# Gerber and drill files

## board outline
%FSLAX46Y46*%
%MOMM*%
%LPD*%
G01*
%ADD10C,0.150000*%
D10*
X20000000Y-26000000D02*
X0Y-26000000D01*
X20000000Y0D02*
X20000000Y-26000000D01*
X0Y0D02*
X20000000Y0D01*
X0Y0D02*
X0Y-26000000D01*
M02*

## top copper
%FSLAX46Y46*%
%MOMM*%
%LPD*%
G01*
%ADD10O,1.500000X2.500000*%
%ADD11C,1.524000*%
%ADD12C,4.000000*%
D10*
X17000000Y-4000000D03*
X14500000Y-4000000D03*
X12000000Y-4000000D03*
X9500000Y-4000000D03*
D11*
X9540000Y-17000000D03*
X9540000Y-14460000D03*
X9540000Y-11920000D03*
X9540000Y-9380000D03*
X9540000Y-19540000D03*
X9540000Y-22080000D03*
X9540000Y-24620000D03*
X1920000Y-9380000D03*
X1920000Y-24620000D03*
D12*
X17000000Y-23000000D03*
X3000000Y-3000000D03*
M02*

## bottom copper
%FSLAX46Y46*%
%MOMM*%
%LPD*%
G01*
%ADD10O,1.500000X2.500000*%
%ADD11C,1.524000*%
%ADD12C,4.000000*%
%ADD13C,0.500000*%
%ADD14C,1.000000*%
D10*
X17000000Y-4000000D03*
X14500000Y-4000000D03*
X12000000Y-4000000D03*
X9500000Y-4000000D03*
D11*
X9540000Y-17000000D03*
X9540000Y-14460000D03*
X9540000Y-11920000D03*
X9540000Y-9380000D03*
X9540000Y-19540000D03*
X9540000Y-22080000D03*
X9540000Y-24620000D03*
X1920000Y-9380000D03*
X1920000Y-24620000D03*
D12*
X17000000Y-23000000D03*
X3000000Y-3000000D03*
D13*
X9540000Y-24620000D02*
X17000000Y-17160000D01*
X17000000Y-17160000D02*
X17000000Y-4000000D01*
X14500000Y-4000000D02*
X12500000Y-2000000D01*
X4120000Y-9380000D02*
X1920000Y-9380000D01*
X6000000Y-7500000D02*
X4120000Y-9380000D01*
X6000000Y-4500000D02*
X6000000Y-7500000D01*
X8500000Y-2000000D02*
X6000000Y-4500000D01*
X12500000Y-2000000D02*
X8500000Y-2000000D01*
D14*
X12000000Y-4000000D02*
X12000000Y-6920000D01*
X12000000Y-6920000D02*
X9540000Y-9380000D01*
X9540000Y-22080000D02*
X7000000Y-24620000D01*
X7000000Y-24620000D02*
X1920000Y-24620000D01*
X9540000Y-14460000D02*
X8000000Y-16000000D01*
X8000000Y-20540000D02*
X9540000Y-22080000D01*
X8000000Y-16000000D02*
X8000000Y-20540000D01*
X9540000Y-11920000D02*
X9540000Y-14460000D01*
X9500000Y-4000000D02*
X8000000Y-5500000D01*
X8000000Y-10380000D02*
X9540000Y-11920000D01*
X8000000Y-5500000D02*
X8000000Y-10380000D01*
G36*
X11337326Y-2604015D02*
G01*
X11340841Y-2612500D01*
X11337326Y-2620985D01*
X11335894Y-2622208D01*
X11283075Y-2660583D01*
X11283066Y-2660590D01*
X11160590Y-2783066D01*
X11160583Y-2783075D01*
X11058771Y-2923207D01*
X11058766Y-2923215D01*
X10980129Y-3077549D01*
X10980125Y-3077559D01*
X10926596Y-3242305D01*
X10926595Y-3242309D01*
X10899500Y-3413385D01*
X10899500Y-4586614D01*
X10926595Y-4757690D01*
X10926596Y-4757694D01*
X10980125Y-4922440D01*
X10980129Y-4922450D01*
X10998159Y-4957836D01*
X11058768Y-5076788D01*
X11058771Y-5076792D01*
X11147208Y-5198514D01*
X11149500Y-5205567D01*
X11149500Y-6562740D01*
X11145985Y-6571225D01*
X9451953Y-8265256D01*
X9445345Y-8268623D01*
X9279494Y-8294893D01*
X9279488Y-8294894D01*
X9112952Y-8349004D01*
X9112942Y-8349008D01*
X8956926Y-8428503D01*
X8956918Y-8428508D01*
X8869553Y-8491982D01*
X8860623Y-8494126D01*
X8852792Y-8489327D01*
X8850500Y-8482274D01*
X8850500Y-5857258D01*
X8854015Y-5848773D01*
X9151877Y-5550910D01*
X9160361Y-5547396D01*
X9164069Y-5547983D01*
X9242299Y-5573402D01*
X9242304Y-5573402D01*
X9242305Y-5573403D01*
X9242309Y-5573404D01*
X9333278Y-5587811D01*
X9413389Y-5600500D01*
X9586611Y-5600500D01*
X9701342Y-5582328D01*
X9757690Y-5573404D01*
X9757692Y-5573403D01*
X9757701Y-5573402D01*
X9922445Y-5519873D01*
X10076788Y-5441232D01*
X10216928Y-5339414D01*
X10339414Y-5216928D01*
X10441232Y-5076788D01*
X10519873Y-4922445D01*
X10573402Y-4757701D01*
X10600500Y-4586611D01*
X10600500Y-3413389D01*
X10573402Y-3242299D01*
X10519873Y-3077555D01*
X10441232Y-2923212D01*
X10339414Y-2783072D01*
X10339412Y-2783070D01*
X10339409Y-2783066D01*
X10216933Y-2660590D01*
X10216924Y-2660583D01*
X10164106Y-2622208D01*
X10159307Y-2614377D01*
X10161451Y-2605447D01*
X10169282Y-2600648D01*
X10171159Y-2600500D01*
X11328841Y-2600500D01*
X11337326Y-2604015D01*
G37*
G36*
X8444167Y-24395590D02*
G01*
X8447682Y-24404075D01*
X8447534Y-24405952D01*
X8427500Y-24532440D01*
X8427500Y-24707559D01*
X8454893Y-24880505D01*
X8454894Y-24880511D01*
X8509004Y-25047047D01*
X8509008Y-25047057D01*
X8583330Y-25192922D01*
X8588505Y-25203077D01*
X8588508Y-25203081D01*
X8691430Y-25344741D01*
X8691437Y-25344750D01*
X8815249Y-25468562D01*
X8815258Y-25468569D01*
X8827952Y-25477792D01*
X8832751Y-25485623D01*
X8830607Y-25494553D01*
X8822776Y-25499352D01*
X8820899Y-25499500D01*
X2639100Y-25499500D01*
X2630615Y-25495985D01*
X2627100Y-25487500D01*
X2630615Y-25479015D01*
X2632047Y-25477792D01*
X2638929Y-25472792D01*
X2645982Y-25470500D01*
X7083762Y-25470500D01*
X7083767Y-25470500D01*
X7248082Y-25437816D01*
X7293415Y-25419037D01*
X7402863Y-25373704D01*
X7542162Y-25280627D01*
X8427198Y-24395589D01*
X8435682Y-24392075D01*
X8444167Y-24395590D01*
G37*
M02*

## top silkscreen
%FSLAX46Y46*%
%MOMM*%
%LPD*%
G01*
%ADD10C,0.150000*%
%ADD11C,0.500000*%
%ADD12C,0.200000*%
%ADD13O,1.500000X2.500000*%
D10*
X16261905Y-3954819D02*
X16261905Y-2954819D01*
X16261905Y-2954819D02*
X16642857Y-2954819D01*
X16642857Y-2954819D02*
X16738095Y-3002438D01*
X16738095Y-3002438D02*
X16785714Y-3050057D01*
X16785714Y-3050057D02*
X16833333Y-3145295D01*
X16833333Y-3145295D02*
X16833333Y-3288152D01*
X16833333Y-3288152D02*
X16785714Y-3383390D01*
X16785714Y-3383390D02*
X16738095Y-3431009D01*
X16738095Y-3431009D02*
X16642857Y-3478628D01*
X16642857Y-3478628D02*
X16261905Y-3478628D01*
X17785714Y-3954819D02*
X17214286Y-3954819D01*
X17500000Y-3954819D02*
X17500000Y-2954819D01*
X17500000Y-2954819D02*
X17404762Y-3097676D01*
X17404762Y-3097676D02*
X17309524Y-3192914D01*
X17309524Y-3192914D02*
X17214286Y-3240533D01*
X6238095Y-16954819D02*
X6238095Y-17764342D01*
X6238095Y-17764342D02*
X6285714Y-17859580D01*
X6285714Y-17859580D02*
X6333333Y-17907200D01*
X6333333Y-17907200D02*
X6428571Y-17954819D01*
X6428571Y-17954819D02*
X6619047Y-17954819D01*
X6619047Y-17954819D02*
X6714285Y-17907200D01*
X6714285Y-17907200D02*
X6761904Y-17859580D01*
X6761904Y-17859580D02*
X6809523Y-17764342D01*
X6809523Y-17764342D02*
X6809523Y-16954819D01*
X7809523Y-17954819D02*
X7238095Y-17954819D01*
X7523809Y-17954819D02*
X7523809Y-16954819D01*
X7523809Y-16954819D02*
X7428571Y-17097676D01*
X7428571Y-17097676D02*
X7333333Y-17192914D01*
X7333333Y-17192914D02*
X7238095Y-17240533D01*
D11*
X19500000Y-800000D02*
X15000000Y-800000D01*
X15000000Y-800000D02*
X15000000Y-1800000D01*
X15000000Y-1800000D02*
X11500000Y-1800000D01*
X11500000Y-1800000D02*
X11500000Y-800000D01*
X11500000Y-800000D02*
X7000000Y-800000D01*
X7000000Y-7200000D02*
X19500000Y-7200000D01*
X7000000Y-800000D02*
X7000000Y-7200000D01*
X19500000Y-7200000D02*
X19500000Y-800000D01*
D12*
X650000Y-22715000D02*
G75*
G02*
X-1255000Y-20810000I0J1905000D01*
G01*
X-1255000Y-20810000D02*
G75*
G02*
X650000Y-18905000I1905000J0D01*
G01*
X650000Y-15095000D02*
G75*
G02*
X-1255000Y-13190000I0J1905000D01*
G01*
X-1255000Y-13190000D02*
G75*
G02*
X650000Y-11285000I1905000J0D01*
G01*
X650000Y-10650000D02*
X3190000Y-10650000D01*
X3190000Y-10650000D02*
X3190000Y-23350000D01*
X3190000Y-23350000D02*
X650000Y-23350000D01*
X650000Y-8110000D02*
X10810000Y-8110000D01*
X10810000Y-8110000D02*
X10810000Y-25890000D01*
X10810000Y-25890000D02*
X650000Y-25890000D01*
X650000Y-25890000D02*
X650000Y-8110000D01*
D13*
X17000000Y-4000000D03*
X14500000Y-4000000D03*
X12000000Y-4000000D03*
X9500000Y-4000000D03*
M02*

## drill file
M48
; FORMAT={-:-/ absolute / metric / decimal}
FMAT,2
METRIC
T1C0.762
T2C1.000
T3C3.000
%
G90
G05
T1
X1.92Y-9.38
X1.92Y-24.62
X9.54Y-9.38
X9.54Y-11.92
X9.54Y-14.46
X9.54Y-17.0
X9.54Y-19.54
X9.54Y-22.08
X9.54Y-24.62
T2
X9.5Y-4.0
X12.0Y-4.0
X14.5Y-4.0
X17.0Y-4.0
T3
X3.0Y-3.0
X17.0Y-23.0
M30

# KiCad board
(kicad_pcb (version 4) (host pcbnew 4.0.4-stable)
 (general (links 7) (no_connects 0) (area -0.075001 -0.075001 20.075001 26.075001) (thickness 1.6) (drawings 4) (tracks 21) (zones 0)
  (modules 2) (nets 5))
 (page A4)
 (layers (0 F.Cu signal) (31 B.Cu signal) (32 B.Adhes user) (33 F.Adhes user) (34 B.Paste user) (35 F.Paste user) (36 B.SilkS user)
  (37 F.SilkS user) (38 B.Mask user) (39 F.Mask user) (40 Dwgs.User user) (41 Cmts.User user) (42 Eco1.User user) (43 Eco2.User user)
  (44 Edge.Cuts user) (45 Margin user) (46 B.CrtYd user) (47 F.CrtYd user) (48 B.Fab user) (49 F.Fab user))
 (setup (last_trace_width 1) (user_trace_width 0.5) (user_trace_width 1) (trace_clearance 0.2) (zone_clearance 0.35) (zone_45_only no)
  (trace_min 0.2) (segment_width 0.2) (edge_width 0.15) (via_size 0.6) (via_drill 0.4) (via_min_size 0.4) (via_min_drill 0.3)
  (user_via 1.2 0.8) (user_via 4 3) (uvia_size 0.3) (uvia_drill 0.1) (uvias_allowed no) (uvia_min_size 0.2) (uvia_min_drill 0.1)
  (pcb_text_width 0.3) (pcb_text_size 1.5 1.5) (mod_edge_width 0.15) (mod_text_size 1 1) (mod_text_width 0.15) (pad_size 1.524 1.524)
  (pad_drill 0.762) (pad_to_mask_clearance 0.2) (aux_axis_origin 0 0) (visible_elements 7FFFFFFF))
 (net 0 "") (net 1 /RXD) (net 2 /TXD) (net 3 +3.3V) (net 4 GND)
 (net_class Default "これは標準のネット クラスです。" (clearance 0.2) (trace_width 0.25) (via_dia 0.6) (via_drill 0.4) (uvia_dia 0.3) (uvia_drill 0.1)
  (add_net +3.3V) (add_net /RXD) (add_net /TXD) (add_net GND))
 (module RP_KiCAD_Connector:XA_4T (layer F.Cu) (at 17 4 180)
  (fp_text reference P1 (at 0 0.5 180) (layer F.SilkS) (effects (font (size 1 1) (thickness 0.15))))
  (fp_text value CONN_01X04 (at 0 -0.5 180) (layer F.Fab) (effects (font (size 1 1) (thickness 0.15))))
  (fp_line (start -2.5 3.2) (end 2 3.2) (layer F.SilkS) (width 0.5))
  (fp_line (start 2 3.2) (end 2 2.2) (layer F.SilkS) (width 0.5))
  (fp_line (start 2 2.2) (end 5.5 2.2) (layer F.SilkS) (width 0.5))
  (fp_line (start 5.5 2.2) (end 5.5 3.2) (layer F.SilkS) (width 0.5))
  (fp_line (start 5.5 3.2) (end 10 3.2) (layer F.SilkS) (width 0.5))
  (fp_line (start 10 -3.2) (end -2.5 -3.2) (layer F.SilkS) (width 0.5))
  (fp_line (start 10 3.2) (end 10 -3.2) (layer F.SilkS) (width 0.5))
  (fp_line (start -2.5 -3.2) (end -2.5 3.2) (layer F.SilkS) (width 0.5))
  (pad 4 thru_hole oval (at 0 0 180) (size 1.5 2.5) (drill 1) (layers *.Cu *.Mask F.SilkS) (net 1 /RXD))
  (pad 3 thru_hole oval (at 2.5 0 180) (size 1.5 2.5) (drill 1) (layers *.Cu *.Mask F.SilkS) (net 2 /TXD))
  (pad 2 thru_hole oval (at 5 0 180) (size 1.5 2.5) (drill 1) (layers *.Cu *.Mask F.SilkS) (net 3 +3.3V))
  (pad 1 thru_hole oval (at 7.5 0 180) (size 1.5 2.5) (drill 1) (layers *.Cu *.Mask F.SilkS) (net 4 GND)))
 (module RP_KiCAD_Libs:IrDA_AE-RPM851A (layer F.Cu) (at 7 17)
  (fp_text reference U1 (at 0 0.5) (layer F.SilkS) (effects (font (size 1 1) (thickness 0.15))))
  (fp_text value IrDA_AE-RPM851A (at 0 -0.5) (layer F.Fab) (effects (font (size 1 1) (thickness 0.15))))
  (fp_arc (start -6.35 3.81) (end -6.35 5.715) (angle 90) (layer F.SilkS) (width 0.2))
  (fp_arc (start -6.35 3.81) (end -8.255 3.81) (angle 90) (layer F.SilkS) (width 0.2))
  (fp_arc (start -6.35 -3.81) (end -6.35 -1.905) (angle 90) (layer F.SilkS) (width 0.2))
  (fp_arc (start -6.35 -3.81) (end -8.255 -3.81) (angle 90) (layer F.SilkS) (width 0.2))
  (fp_line (start -6.35 -6.35) (end -3.81 -6.35) (layer F.SilkS) (width 0.2))
  (fp_line (start -3.81 -6.35) (end -3.81 6.35) (layer F.SilkS) (width 0.2))
  (fp_line (start -3.81 6.35) (end -6.35 6.35) (layer F.SilkS) (width 0.2))
  (fp_line (start -6.35 -8.89) (end 3.81 -8.89) (layer F.SilkS) (width 0.2))
  (fp_line (start 3.81 -8.89) (end 3.81 8.89) (layer F.SilkS) (width 0.2))
  (fp_line (start 3.81 8.89) (end -6.35 8.89) (layer F.SilkS) (width 0.2))
  (fp_line (start -6.35 8.89) (end -6.35 -8.89) (layer F.SilkS) (width 0.2))
  (pad 11 thru_hole circle (at 2.54 0) (size 1.524 1.524) (drill 0.762) (layers *.Cu *.Mask))
  (pad 12 thru_hole circle (at 2.54 -2.54) (size 1.524 1.524) (drill 0.762) (layers *.Cu *.Mask) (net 4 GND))
  (pad 13 thru_hole circle (at 2.54 -5.08) (size 1.524 1.524) (drill 0.762) (layers *.Cu *.Mask) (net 4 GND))
  (pad 14 thru_hole circle (at 2.54 -7.62) (size 1.524 1.524) (drill 0.762) (layers *.Cu *.Mask) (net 3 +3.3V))
  (pad 10 thru_hole circle (at 2.54 2.54) (size 1.524 1.524) (drill 0.762) (layers *.Cu *.Mask))
  (pad 9 thru_hole circle (at 2.54 5.08) (size 1.524 1.524) (drill 0.762) (layers *.Cu *.Mask) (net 4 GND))
  (pad 8 thru_hole circle (at 2.54 7.62) (size 1.524 1.524) (drill 0.762) (layers *.Cu *.Mask) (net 1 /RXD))
  (pad 1 thru_hole circle (at -5.08 -7.62) (size 1.524 1.524) (drill 0.762) (layers *.Cu *.Mask) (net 2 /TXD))
  (pad 7 thru_hole circle (at -5.08 7.62) (size 1.524 1.524) (drill 0.762) (layers *.Cu *.Mask) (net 4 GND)))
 (gr_line (start 20 26) (end 0 26) (angle 90) (layer Edge.Cuts) (width 0.15))
 (gr_line (start 20 0) (end 20 26) (angle 90) (layer Edge.Cuts) (width 0.15))
 (gr_line (start 0 0) (end 20 0) (angle 90) (layer Edge.Cuts) (width 0.15))
 (gr_line (start 0 0) (end 0 26) (angle 90) (layer Edge.Cuts) (width 0.15))
 (via (at 17 23) (size 4) (drill 3) (layers F.Cu B.Cu) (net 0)) (via (at 3 3) (size 4) (drill 3) (layers F.Cu B.Cu) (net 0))
 (segment (start 9.54 24.62) (end 17 17.16) (width 0.5) (layer B.Cu) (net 1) (status 400000))
 (segment (start 17 17.16) (end 17 4) (width 0.5) (layer B.Cu) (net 1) (status 800000))
 (segment (start 14.5 4) (end 12.5 2) (width 0.5) (layer B.Cu) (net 2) (status 400000))
 (segment (start 4.12 9.38) (end 1.92 9.38) (width 0.5) (layer B.Cu) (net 2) (status 800000))
 (segment (start 6 7.5) (end 4.12 9.38) (width 0.5) (layer B.Cu) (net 2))
 (segment (start 6 4.5) (end 6 7.5) (width 0.5) (layer B.Cu) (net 2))
 (segment (start 8.5 2) (end 6 4.5) (width 0.5) (layer B.Cu) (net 2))
 (segment (start 12.5 2) (end 8.5 2) (width 0.5) (layer B.Cu) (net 2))
 (segment (start 12 4) (end 12 6.92) (width 1) (layer B.Cu) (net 3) (status 400000))
 (segment (start 12 6.92) (end 9.54 9.38) (width 1) (layer B.Cu) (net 3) (status 800000))
 (segment (start 9.54 22.08) (end 7 24.62) (width 1) (layer B.Cu) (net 4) (status 400000))
 (segment (start 7 24.62) (end 1.92 24.62) (width 1) (layer B.Cu) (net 4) (status 800000))
 (segment (start 9.54 14.46) (end 8 16) (width 1) (layer B.Cu) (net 4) (status 400000))
 (segment (start 8 20.54) (end 9.54 22.08) (width 1) (layer B.Cu) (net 4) (status 800000))
 (segment (start 8 16) (end 8 20.54) (width 1) (layer B.Cu) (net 4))
 (segment (start 9.54 11.92) (end 9.54 14.46) (width 1) (layer B.Cu) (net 4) (status C00000))
 (segment (start 9.5 4) (end 8 5.5) (width 1) (layer B.Cu) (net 4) (status 400000))
 (segment (start 8 10.38) (end 9.54 11.92) (width 1) (layer B.Cu) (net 4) (status 800000))
 (segment (start 8 5.5) (end 8 10.38) (width 1) (layer B.Cu) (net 4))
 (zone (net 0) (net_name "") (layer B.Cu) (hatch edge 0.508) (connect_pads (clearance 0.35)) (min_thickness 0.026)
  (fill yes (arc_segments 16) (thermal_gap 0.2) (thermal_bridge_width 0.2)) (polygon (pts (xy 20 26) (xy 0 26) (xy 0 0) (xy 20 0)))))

